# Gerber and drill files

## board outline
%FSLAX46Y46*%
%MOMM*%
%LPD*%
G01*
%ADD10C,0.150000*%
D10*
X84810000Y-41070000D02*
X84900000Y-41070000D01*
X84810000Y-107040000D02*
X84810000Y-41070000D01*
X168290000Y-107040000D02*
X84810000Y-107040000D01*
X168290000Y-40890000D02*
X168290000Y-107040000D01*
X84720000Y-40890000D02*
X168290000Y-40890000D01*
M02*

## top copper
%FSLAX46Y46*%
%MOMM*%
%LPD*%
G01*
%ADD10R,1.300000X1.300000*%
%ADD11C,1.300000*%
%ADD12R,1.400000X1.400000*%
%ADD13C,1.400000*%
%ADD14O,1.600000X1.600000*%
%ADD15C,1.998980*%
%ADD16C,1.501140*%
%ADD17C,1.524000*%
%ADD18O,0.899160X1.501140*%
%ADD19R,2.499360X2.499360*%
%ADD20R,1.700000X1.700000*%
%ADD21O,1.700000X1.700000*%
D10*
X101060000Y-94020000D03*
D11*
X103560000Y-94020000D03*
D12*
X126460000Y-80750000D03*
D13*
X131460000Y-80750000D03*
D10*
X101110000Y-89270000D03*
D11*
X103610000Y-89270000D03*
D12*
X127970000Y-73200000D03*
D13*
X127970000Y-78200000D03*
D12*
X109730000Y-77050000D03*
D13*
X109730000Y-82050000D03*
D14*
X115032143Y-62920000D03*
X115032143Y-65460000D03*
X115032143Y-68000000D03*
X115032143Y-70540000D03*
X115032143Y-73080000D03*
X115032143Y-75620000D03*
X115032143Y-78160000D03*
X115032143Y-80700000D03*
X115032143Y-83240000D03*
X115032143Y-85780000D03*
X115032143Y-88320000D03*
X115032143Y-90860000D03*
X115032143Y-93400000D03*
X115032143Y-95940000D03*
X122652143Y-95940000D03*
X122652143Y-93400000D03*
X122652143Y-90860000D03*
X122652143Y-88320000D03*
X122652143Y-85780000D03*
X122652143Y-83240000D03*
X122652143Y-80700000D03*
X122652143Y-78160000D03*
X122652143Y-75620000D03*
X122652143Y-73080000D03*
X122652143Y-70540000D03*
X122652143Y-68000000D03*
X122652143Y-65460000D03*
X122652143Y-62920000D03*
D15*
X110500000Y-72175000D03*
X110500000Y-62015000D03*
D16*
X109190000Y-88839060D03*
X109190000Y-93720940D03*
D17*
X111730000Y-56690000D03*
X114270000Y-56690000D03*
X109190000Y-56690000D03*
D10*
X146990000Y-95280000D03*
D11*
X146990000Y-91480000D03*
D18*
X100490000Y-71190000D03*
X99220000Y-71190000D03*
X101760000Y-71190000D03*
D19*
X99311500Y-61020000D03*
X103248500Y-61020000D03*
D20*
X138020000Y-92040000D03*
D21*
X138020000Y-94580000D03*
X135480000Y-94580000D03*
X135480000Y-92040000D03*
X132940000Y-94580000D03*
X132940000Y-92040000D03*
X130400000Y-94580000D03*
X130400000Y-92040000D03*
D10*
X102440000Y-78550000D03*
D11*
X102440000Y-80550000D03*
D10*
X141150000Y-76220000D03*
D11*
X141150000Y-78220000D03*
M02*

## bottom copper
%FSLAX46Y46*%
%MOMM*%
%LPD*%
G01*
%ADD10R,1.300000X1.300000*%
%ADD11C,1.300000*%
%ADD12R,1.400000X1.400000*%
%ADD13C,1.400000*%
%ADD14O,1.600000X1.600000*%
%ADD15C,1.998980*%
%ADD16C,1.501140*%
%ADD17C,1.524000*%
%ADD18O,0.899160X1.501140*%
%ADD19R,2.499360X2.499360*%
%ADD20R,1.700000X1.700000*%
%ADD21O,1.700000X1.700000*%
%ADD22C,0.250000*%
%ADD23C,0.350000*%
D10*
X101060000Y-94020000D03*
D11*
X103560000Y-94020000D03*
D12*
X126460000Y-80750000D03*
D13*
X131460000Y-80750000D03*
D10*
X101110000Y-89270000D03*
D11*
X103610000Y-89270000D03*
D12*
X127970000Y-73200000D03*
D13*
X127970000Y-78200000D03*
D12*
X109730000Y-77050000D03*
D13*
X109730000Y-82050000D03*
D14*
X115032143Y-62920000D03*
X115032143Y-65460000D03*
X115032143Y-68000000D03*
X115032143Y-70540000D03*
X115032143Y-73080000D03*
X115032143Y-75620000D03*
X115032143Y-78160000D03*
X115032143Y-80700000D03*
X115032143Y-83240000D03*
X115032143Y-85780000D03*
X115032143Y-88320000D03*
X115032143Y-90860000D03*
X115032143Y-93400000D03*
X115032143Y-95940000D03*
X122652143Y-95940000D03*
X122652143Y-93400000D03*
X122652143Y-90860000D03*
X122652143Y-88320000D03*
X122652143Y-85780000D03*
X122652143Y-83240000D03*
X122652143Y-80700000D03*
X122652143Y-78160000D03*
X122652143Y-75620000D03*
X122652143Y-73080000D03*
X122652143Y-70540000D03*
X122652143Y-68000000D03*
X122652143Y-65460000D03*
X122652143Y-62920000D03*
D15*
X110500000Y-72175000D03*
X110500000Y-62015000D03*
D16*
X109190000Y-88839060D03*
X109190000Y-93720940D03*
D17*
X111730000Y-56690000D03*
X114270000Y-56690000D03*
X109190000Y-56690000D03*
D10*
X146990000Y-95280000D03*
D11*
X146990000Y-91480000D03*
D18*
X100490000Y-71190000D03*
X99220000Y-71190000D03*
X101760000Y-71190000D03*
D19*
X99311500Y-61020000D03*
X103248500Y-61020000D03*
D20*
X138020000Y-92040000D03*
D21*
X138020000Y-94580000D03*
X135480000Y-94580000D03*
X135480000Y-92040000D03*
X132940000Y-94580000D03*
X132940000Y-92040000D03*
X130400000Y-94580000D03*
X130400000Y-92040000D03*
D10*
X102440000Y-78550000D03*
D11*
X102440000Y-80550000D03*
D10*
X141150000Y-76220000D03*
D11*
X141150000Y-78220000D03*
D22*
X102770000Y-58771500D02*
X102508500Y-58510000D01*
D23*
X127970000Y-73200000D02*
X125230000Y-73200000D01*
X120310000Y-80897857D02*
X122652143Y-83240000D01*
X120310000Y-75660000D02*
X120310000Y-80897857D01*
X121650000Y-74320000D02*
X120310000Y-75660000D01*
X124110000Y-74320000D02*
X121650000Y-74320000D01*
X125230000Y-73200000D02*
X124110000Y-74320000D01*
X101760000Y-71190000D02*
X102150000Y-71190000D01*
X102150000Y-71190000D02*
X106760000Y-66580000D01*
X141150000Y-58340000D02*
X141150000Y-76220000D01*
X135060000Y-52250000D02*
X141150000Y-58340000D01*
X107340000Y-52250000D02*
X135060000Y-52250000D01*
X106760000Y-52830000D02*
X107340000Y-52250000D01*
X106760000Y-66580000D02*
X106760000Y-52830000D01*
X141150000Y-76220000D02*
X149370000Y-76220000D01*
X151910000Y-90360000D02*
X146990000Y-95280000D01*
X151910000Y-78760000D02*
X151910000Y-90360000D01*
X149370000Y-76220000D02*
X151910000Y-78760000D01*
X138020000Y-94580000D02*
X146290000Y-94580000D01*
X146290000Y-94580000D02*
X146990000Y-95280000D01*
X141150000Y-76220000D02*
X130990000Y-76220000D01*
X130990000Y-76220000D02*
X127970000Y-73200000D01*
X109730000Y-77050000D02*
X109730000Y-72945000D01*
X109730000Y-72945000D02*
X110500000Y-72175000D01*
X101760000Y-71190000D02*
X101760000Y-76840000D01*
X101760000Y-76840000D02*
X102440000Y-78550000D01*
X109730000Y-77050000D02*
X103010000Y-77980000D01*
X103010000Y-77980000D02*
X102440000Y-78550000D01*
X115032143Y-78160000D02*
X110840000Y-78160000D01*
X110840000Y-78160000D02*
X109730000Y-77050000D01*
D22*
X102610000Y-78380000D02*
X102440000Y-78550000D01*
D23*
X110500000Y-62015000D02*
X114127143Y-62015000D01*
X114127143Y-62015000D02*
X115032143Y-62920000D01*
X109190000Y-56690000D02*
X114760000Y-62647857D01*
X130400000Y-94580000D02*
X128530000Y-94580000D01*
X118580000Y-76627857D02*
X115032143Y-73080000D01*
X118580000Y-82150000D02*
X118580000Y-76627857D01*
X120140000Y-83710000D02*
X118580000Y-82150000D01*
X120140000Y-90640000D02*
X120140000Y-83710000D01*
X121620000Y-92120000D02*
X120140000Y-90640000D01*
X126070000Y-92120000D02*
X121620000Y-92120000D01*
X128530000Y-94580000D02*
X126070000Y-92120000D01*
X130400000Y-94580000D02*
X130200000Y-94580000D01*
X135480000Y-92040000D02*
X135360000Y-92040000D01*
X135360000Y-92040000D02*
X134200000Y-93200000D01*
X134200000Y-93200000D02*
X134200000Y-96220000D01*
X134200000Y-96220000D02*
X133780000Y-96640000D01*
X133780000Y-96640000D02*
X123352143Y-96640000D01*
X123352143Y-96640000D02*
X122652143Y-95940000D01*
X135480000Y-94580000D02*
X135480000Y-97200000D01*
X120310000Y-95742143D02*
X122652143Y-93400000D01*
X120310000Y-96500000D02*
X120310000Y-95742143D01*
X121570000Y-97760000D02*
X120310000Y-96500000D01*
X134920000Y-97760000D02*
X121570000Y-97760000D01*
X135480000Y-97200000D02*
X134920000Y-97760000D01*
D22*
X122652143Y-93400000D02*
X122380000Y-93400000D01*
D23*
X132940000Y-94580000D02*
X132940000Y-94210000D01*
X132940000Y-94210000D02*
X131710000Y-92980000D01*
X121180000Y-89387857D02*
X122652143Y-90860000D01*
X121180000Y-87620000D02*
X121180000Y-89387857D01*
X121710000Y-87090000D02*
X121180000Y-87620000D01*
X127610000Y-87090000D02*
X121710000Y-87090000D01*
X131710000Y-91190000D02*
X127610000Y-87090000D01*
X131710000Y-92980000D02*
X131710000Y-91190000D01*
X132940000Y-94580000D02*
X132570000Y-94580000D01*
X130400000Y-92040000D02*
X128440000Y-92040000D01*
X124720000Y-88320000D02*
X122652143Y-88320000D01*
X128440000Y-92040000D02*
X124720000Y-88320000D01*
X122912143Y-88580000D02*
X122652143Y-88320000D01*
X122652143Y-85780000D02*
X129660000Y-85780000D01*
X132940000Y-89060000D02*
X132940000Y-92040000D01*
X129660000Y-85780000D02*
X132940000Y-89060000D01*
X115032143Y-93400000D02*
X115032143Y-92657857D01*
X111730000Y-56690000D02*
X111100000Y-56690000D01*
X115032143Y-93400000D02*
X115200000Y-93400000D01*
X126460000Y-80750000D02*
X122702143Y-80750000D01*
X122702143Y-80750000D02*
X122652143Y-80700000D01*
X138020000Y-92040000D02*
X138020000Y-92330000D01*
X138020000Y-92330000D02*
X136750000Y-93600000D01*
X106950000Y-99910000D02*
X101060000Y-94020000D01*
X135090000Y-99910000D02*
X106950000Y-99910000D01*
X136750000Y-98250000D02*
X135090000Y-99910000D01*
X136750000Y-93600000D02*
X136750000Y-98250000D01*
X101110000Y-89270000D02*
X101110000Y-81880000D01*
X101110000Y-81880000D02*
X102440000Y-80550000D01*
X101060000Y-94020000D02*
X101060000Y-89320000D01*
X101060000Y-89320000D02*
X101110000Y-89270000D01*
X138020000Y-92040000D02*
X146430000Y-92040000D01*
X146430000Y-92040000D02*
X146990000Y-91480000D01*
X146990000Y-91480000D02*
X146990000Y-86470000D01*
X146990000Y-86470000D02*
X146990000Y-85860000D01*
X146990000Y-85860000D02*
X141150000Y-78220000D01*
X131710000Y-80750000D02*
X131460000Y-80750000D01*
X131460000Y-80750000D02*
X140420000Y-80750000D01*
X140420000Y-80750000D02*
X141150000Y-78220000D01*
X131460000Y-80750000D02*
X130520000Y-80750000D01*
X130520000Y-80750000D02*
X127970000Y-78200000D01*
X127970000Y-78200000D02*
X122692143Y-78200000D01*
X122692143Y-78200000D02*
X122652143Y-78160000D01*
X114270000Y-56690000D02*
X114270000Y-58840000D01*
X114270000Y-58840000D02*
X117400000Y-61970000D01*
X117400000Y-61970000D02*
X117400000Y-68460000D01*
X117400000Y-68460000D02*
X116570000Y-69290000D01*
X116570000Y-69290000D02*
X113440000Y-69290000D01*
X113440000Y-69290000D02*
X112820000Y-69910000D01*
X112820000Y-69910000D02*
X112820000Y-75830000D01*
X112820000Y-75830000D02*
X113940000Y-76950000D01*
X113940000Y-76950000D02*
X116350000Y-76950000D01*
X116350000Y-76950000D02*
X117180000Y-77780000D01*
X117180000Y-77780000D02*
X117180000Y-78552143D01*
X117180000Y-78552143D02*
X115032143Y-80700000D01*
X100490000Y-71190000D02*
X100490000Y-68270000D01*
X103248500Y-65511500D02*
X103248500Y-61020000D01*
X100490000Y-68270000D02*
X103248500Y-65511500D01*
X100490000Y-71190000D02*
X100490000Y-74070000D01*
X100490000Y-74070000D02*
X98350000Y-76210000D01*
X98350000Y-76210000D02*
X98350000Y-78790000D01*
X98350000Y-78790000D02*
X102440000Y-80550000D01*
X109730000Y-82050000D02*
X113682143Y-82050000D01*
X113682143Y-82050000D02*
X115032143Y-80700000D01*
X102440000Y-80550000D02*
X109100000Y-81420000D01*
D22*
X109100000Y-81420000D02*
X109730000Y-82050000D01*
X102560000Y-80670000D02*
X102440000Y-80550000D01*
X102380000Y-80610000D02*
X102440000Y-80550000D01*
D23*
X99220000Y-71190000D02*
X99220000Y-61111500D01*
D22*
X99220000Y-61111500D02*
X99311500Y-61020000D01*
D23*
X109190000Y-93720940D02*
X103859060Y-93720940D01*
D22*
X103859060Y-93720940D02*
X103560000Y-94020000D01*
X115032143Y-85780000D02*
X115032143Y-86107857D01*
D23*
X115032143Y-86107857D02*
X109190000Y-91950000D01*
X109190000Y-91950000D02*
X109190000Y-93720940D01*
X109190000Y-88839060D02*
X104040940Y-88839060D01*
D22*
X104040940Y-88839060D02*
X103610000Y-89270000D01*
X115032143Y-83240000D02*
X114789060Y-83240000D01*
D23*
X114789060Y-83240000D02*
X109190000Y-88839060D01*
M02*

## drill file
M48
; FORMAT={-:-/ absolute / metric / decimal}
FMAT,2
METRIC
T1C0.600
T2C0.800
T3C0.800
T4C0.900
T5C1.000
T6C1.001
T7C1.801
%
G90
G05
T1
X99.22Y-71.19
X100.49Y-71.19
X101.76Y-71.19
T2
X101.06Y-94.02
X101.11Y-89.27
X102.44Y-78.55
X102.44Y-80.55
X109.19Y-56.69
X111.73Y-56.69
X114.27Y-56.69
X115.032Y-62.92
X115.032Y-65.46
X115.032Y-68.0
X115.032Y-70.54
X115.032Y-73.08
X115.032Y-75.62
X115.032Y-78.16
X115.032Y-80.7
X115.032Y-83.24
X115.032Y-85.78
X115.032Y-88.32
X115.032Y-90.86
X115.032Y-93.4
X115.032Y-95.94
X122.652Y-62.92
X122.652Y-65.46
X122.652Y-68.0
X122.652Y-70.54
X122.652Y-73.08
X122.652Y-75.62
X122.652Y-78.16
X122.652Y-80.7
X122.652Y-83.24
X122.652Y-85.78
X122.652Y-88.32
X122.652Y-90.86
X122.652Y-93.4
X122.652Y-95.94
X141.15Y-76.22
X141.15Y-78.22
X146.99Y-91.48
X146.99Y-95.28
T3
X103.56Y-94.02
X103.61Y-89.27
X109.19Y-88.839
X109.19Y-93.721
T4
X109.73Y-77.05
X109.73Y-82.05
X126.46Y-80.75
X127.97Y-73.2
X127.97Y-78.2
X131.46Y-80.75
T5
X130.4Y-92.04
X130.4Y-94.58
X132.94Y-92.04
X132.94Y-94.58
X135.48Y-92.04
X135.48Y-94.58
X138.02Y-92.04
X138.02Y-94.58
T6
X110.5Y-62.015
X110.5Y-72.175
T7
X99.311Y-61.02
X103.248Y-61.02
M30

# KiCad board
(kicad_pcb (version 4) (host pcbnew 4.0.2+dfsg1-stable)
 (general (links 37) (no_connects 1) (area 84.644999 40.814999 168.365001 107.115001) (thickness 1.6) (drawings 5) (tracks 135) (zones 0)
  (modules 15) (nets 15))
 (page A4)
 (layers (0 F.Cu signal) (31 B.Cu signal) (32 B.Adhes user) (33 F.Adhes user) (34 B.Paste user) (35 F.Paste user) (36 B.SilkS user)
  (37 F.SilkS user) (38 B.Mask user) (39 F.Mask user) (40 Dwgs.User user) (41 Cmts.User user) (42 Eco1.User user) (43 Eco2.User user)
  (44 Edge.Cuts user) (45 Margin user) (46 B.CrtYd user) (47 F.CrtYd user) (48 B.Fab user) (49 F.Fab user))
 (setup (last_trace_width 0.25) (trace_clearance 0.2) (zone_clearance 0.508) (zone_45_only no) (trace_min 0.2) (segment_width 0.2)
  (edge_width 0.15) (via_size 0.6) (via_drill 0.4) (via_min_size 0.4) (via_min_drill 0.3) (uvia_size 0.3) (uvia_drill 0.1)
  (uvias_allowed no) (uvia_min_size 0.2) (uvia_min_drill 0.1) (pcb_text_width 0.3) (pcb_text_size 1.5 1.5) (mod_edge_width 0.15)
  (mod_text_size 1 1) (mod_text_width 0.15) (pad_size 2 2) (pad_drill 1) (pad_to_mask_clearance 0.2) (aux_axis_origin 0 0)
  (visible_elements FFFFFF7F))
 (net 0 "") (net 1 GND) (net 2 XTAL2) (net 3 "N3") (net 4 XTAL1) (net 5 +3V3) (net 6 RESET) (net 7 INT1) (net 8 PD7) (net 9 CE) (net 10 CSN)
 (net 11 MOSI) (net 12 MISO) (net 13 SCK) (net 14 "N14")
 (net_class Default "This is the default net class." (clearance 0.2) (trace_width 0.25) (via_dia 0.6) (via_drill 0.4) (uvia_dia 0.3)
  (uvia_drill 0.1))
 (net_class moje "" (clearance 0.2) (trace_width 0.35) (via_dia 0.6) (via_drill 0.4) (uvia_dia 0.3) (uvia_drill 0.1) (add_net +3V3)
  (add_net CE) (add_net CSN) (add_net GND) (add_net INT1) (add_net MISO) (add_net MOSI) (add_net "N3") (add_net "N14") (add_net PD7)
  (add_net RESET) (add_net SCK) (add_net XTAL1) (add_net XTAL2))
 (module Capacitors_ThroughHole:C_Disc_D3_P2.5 (layer F.Cu) (at 101.06 94.02)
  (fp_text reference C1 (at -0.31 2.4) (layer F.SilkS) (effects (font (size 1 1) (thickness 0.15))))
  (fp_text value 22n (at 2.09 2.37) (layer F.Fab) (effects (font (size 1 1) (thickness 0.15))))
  (pad 1 thru_hole rect (at 0 0) (size 1.3 1.3) (drill 0.8) (layers *.Cu *.Mask F.SilkS) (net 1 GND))
  (pad 2 thru_hole circle (at 2.5 0) (size 1.3 1.3) (drill 0.8001) (layers *.Cu *.Mask F.SilkS) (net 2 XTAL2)))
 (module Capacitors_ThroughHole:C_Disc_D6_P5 (layer F.Cu) (at 126.46 80.75)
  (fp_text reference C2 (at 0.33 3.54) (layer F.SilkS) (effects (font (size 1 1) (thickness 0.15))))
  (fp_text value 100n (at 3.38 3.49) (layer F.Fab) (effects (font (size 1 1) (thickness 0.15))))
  (pad 1 thru_hole rect (at 0 0) (size 1.4 1.4) (drill 0.9) (layers *.Cu *.Mask F.SilkS) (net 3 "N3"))
  (pad 2 thru_hole circle (at 5 0) (size 1.4 1.4) (drill 0.9) (layers *.Cu *.Mask F.SilkS) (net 1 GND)))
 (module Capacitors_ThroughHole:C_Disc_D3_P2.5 (layer F.Cu) (at 101.11 89.27)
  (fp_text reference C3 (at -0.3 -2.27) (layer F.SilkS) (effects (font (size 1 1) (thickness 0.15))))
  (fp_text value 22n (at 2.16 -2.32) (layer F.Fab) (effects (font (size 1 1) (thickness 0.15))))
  (pad 1 thru_hole rect (at 0 0) (size 1.3 1.3) (drill 0.8) (layers *.Cu *.Mask F.SilkS) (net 1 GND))
  (pad 2 thru_hole circle (at 2.5 0) (size 1.3 1.3) (drill 0.8001) (layers *.Cu *.Mask F.SilkS) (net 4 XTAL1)))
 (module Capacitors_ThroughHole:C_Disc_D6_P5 (layer F.Cu) (at 127.97 73.2 270)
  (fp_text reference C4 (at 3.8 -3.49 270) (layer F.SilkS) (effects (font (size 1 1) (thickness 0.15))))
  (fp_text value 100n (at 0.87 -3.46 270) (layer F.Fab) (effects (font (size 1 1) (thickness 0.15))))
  (pad 1 thru_hole rect (at 0 0 270) (size 1.4 1.4) (drill 0.9) (layers *.Cu *.Mask F.SilkS) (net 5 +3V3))
  (pad 2 thru_hole circle (at 5 0 270) (size 1.4 1.4) (drill 0.9) (layers *.Cu *.Mask F.SilkS) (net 1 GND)))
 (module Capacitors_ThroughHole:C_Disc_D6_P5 (layer F.Cu) (at 109.73 77.05 270)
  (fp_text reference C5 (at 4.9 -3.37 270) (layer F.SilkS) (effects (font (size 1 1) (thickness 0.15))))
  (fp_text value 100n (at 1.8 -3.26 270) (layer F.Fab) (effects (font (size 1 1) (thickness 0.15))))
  (pad 1 thru_hole rect (at 0 0 270) (size 1.4 1.4) (drill 0.9) (layers *.Cu *.Mask F.SilkS) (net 5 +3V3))
  (pad 2 thru_hole circle (at 5 0 270) (size 1.4 1.4) (drill 0.9) (layers *.Cu *.Mask F.SilkS) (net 1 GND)))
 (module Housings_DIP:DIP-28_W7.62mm (layer F.Cu) (at 115.032143 62.92)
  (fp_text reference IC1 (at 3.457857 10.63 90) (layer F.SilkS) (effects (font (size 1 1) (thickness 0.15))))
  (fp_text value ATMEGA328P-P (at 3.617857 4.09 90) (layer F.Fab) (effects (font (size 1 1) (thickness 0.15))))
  (pad 1 thru_hole oval (at 0 0) (size 1.6 1.6) (drill 0.8) (layers *.Cu *.Mask F.SilkS) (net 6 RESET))
  (pad 2 thru_hole oval (at 0 2.54) (size 1.6 1.6) (drill 0.8) (layers *.Cu *.Mask F.SilkS))
  (pad 3 thru_hole oval (at 0 5.08) (size 1.6 1.6) (drill 0.8) (layers *.Cu *.Mask F.SilkS))
  (pad 4 thru_hole oval (at 0 7.62) (size 1.6 1.6) (drill 0.8) (layers *.Cu *.Mask F.SilkS))
  (pad 5 thru_hole oval (at 0 10.16) (size 1.6 1.6) (drill 0.8) (layers *.Cu *.Mask F.SilkS) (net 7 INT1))
  (pad 6 thru_hole oval (at 0 12.7) (size 1.6 1.6) (drill 0.8) (layers *.Cu *.Mask F.SilkS))
  (pad 7 thru_hole oval (at 0 15.24) (size 1.6 1.6) (drill 0.8) (layers *.Cu *.Mask F.SilkS) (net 5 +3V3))
  (pad 8 thru_hole oval (at 0 17.78) (size 1.6 1.6) (drill 0.8) (layers *.Cu *.Mask F.SilkS) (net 1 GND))
  (pad 9 thru_hole oval (at 0 20.32) (size 1.6 1.6) (drill 0.8) (layers *.Cu *.Mask F.SilkS) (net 4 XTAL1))
  (pad 10 thru_hole oval (at 0 22.86) (size 1.6 1.6) (drill 0.8) (layers *.Cu *.Mask F.SilkS) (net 2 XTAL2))
  (pad 11 thru_hole oval (at 0 25.4) (size 1.6 1.6) (drill 0.8) (layers *.Cu *.Mask F.SilkS))
  (pad 12 thru_hole oval (at 0 27.94) (size 1.6 1.6) (drill 0.8) (layers *.Cu *.Mask F.SilkS))
  (pad 13 thru_hole oval (at 0 30.48) (size 1.6 1.6) (drill 0.8) (layers *.Cu *.Mask F.SilkS) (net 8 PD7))
  (pad 14 thru_hole oval (at 0 33.02) (size 1.6 1.6) (drill 0.8) (layers *.Cu *.Mask F.SilkS))
  (pad 15 thru_hole oval (at 7.62 33.02) (size 1.6 1.6) (drill 0.8) (layers *.Cu *.Mask F.SilkS) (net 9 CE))
  (pad 16 thru_hole oval (at 7.62 30.48) (size 1.6 1.6) (drill 0.8) (layers *.Cu *.Mask F.SilkS) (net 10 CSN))
  (pad 17 thru_hole oval (at 7.62 27.94) (size 1.6 1.6) (drill 0.8) (layers *.Cu *.Mask F.SilkS) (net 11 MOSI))
  (pad 18 thru_hole oval (at 7.62 25.4) (size 1.6 1.6) (drill 0.8) (layers *.Cu *.Mask F.SilkS) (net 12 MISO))
  (pad 19 thru_hole oval (at 7.62 22.86) (size 1.6 1.6) (drill 0.8) (layers *.Cu *.Mask F.SilkS) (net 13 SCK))
  (pad 20 thru_hole oval (at 7.62 20.32) (size 1.6 1.6) (drill 0.8) (layers *.Cu *.Mask F.SilkS) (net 5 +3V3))
  (pad 21 thru_hole oval (at 7.62 17.78) (size 1.6 1.6) (drill 0.8) (layers *.Cu *.Mask F.SilkS) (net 3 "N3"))
  (pad 22 thru_hole oval (at 7.62 15.24) (size 1.6 1.6) (drill 0.8) (layers *.Cu *.Mask F.SilkS) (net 1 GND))
  (pad 23 thru_hole oval (at 7.62 12.7) (size 1.6 1.6) (drill 0.8) (layers *.Cu *.Mask F.SilkS))
  (pad 24 thru_hole oval (at 7.62 10.16) (size 1.6 1.6) (drill 0.8) (layers *.Cu *.Mask F.SilkS))
  (pad 25 thru_hole oval (at 7.62 7.62) (size 1.6 1.6) (drill 0.8) (layers *.Cu *.Mask F.SilkS))
  (pad 26 thru_hole oval (at 7.62 5.08) (size 1.6 1.6) (drill 0.8) (layers *.Cu *.Mask F.SilkS))
  (pad 27 thru_hole oval (at 7.62 2.54) (size 1.6 1.6) (drill 0.8) (layers *.Cu *.Mask F.SilkS))
  (pad 28 thru_hole oval (at 7.62 0) (size 1.6 1.6) (drill 0.8) (layers *.Cu *.Mask F.SilkS)))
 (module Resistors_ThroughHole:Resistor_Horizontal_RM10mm (layer F.Cu) (at 110.5 72.175 90)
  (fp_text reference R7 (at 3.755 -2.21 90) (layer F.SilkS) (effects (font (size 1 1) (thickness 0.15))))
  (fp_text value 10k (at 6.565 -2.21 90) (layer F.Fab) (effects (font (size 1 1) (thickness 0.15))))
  (pad 1 thru_hole circle (at 0 0 90) (size 1.99898 1.99898) (drill 1.00076) (layers *.Cu *.SilkS *.Mask) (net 5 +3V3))
  (pad 2 thru_hole circle (at 10.16 0 90) (size 1.99898 1.99898) (drill 1.00076) (layers *.Cu *.SilkS *.Mask) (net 6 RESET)))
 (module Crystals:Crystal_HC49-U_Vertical (layer F.Cu) (at 109.19 91.28 270)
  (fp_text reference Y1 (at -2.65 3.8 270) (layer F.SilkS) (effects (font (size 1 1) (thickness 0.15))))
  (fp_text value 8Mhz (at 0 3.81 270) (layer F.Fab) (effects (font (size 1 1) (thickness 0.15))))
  (pad 1 thru_hole circle (at -2.44094 0 270) (size 1.50114 1.50114) (drill 0.8001) (layers *.Cu *.Mask F.SilkS) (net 4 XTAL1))
  (pad 2 thru_hole circle (at 2.44094 0 270) (size 1.50114 1.50114) (drill 0.8001) (layers *.Cu *.Mask F.SilkS) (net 2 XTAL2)))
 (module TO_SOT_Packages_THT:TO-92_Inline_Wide (layer F.Cu) (at 109.19 56.69)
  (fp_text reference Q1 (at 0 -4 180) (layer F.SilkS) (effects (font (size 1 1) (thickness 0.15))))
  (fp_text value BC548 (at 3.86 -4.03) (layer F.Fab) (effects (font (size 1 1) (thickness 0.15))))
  (pad 2 thru_hole circle (at 2.54 0 90) (size 1.524 1.524) (drill 0.8) (layers *.Cu *.Mask F.SilkS) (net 8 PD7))
  (pad 3 thru_hole circle (at 5.08 0 90) (size 1.524 1.524) (drill 0.8) (layers *.Cu *.Mask F.SilkS) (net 1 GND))
  (pad 1 thru_hole circle (at 0 0 90) (size 1.524 1.524) (drill 0.8) (layers *.Cu *.Mask F.SilkS) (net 6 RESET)))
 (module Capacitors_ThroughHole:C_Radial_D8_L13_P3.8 (layer F.Cu) (at 146.99 95.28 90)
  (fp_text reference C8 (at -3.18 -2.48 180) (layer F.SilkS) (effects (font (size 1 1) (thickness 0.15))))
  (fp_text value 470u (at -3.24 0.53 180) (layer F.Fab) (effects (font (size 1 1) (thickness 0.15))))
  (pad 1 thru_hole rect (at 0 0 90) (size 1.3 1.3) (drill 0.8) (layers *.Cu *.Mask F.SilkS) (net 5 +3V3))
  (pad 2 thru_hole circle (at 3.8 0 90) (size 1.3 1.3) (drill 0.8) (layers *.Cu *.Mask F.SilkS) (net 1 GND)))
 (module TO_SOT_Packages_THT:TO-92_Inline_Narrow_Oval (layer F.Cu) (at 101.76 71.19 180)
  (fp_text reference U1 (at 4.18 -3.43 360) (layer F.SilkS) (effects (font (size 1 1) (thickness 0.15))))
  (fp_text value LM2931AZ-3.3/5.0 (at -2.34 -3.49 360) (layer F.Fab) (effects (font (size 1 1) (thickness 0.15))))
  (pad 2 thru_hole oval (at 1.27 0) (size 0.89916 1.50114) (drill 0.6) (layers *.Cu *.Mask F.SilkS) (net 1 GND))
  (pad 3 thru_hole oval (at 2.54 0) (size 0.89916 1.50114) (drill 0.6) (layers *.Cu *.Mask F.SilkS) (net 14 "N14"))
  (pad 1 thru_hole oval (at 0 0) (size 0.89916 1.50114) (drill 0.6) (layers *.Cu *.Mask F.SilkS) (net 5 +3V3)))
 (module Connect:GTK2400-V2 (layer F.Cu) (at 101.28 61.02 180)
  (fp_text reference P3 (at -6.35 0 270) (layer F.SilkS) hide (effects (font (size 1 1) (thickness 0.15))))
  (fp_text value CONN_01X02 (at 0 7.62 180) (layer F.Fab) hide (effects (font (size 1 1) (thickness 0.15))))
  (pad 2 thru_hole rect (at 1.9685 0 180) (size 2.49936 2.49936) (drill 1.80086) (layers *.Cu *.Mask F.SilkS) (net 14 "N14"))
  (pad 1 thru_hole rect (at -1.9685 0 180) (size 2.49936 2.49936) (drill 1.80086) (layers *.Cu *.Mask F.SilkS) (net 1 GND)))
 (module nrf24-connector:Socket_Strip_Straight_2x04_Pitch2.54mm (layer F.Cu) (at 138.02 94.58 270)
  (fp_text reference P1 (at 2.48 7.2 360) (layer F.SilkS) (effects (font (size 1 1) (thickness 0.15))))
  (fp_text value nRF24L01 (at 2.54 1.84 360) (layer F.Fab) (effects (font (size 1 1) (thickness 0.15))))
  (pad 1 thru_hole rect (at -2.54 0 270) (size 1.7 1.7) (drill 1) (layers *.Cu *.Mask) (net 1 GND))
  (pad 2 thru_hole oval (at 0 0 270) (size 1.7 1.7) (drill 1) (layers *.Cu *.Mask) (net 5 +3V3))
  (pad 4 thru_hole oval (at 0 2.54 270) (size 1.7 1.7) (drill 1) (layers *.Cu *.Mask) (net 10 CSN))
  (pad 3 thru_hole oval (at -2.54 2.54 270) (size 1.7 1.7) (drill 1) (layers *.Cu *.Mask) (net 9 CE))
  (pad 6 thru_hole oval (at 0 5.08 270) (size 1.7 1.7) (drill 1) (layers *.Cu *.Mask) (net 11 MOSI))
  (pad 5 thru_hole oval (at -2.54 5.08 270) (size 1.7 1.7) (drill 1) (layers *.Cu *.Mask) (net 13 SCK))
  (pad 8 thru_hole oval (at 0 7.62 270) (size 1.7 1.7) (drill 1) (layers *.Cu *.Mask) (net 7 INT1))
  (pad 7 thru_hole oval (at -2.54 7.62 270) (size 1.7 1.7) (drill 1) (layers *.Cu *.Mask) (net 12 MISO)))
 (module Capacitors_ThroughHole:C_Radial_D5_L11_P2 (layer F.Cu) (at 102.44 78.55 270)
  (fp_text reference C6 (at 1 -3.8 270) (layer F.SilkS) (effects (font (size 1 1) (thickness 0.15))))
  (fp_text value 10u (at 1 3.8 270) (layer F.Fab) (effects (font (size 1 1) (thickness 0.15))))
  (pad 1 thru_hole rect (at 0 0 270) (size 1.3 1.3) (drill 0.8) (layers *.Cu *.Mask F.SilkS) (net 5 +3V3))
  (pad 2 thru_hole circle (at 2 0 270) (size 1.3 1.3) (drill 0.8) (layers *.Cu *.Mask F.SilkS) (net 1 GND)))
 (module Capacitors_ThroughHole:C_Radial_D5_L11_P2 (layer F.Cu) (at 141.15 76.22 270)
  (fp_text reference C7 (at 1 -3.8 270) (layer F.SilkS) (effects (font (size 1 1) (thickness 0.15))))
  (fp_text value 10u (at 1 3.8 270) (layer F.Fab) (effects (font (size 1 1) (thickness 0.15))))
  (pad 1 thru_hole rect (at 0 0 270) (size 1.3 1.3) (drill 0.8) (layers *.Cu *.Mask F.SilkS) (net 5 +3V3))
  (pad 2 thru_hole circle (at 2 0 270) (size 1.3 1.3) (drill 0.8) (layers *.Cu *.Mask F.SilkS) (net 1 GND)))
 (gr_line (start 84.81 41.07) (end 84.9 41.07) (angle 90) (layer Edge.Cuts) (width 0.15))
 (gr_line (start 84.81 107.04) (end 84.81 41.07) (angle 90) (layer Edge.Cuts) (width 0.15))
 (gr_line (start 168.29 107.04) (end 84.81 107.04) (angle 90) (layer Edge.Cuts) (width 0.15))
 (gr_line (start 168.29 40.89) (end 168.29 107.04) (angle 90) (layer Edge.Cuts) (width 0.15))
 (gr_line (start 84.72 40.89) (end 168.29 40.89) (angle 90) (layer Edge.Cuts) (width 0.15))
 (segment (start 102.77 58.7715) (end 102.5085 58.51) (width 0.25) (layer B.Cu) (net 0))
 (segment (start 127.97 73.2) (end 125.23 73.2) (width 0.35) (layer B.Cu) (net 5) (status 400000))
 (segment (start 120.31 80.897857) (end 122.652143 83.24) (width 0.35) (layer B.Cu) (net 5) (status 800000))
 (segment (start 120.31 75.66) (end 120.31 80.897857) (width 0.35) (layer B.Cu) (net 5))
 (segment (start 121.65 74.32) (end 120.31 75.66) (width 0.35) (layer B.Cu) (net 5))
 (segment (start 124.11 74.32) (end 121.65 74.32) (width 0.35) (layer B.Cu) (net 5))
 (segment (start 125.23 73.2) (end 124.11 74.32) (width 0.35) (layer B.Cu) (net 5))
 (segment (start 101.76 71.19) (end 102.15 71.19) (width 0.35) (layer B.Cu) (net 5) (status C00000))
 (segment (start 102.15 71.19) (end 106.76 66.58) (width 0.35) (layer B.Cu) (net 5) (status 400000))
 (segment (start 141.15 58.34) (end 141.15 76.22) (width 0.35) (layer B.Cu) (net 5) (status 800000))
 (segment (start 135.06 52.25) (end 141.15 58.34) (width 0.35) (layer B.Cu) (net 5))
 (segment (start 107.34 52.25) (end 135.06 52.25) (width 0.35) (layer B.Cu) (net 5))
 (segment (start 106.76 52.83) (end 107.34 52.25) (width 0.35) (layer B.Cu) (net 5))
 (segment (start 106.76 66.58) (end 106.76 52.83) (width 0.35) (layer B.Cu) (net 5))
 (segment (start 141.15 76.22) (end 149.37 76.22) (width 0.35) (layer B.Cu) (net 5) (status 400000))
 (segment (start 151.91 90.36) (end 146.99 95.28) (width 0.35) (layer B.Cu) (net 5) (status 800000))
 (segment (start 151.91 78.76) (end 151.91 90.36) (width 0.35) (layer B.Cu) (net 5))
 (segment (start 149.37 76.22) (end 151.91 78.76) (width 0.35) (layer B.Cu) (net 5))
 (segment (start 138.02 94.58) (end 146.29 94.58) (width 0.35) (layer B.Cu) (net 5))
 (segment (start 146.29 94.58) (end 146.99 95.28) (width 0.35) (layer B.Cu) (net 5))
 (segment (start 141.15 76.22) (end 130.99 76.22) (width 0.35) (layer B.Cu) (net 5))
 (segment (start 130.99 76.22) (end 127.97 73.2) (width 0.35) (layer B.Cu) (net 5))
 (segment (start 109.73 77.05) (end 109.73 72.945) (width 0.35) (layer B.Cu) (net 5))
 (segment (start 109.73 72.945) (end 110.5 72.175) (width 0.35) (layer B.Cu) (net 5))
 (segment (start 101.76 71.19) (end 101.76 76.84) (width 0.35) (layer B.Cu) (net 5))
 (segment (start 101.76 76.84) (end 102.44 78.55) (width 0.35) (layer B.Cu) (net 5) (status 20))
 (segment (start 109.73 77.05) (end 103.01 77.98) (width 0.35) (layer B.Cu) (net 5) (status 20))
 (segment (start 103.01 77.98) (end 102.44 78.55) (width 0.35) (layer B.Cu) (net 5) (status 30))
 (segment (start 115.032143 78.16) (end 110.84 78.16) (width 0.35) (layer B.Cu) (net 5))
 (segment (start 110.84 78.16) (end 109.73 77.05) (width 0.35) (layer B.Cu) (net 5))
 (segment (start 102.61 78.38) (end 102.44 78.55) (width 0.25) (layer B.Cu) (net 5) (status 30))
 (segment (start 110.5 62.015) (end 114.127143 62.015) (width 0.35) (layer B.Cu) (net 6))
 (segment (start 114.127143 62.015) (end 115.032143 62.92) (width 0.35) (layer B.Cu) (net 6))
 (segment (start 109.19 56.69) (end 114.76 62.647857) (width 0.35) (layer B.Cu) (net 6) (status 10))
 (segment (start 130.4 94.58) (end 128.53 94.58) (width 0.35) (layer B.Cu) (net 7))
 (segment (start 118.58 76.627857) (end 115.032143 73.08) (width 0.35) (layer B.Cu) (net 7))
 (segment (start 118.58 82.15) (end 118.58 76.627857) (width 0.35) (layer B.Cu) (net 7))
 (segment (start 120.14 83.71) (end 118.58 82.15) (width 0.35) (layer B.Cu) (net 7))
 (segment (start 120.14 90.64) (end 120.14 83.71) (width 0.35) (layer B.Cu) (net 7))
 (segment (start 121.62 92.12) (end 120.14 90.64) (width 0.35) (layer B.Cu) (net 7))
 (segment (start 126.07 92.12) (end 121.62 92.12) (width 0.35) (layer B.Cu) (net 7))
 (segment (start 128.53 94.58) (end 126.07 92.12) (width 0.35) (layer B.Cu) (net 7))
 (segment (start 130.4 94.58) (end 130.2 94.58) (width 0.35) (layer B.Cu) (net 7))
 (segment (start 135.48 92.04) (end 135.36 92.04) (width 0.35) (layer B.Cu) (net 9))
 (segment (start 135.36 92.04) (end 134.2 93.2) (width 0.35) (layer B.Cu) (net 9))
 (segment (start 134.2 93.2) (end 134.2 96.22) (width 0.35) (layer B.Cu) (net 9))
 (segment (start 134.2 96.22) (end 133.78 96.64) (width 0.35) (layer B.Cu) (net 9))
 (segment (start 133.78 96.64) (end 123.352143 96.64) (width 0.35) (layer B.Cu) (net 9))
 (segment (start 123.352143 96.64) (end 122.652143 95.94) (width 0.35) (layer B.Cu) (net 9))
 (segment (start 135.48 94.58) (end 135.48 97.2) (width 0.35) (layer B.Cu) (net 10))
 (segment (start 120.31 95.742143) (end 122.652143 93.4) (width 0.35) (layer B.Cu) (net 10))
 (segment (start 120.31 96.5) (end 120.31 95.742143) (width 0.35) (layer B.Cu) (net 10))
 (segment (start 121.57 97.76) (end 120.31 96.5) (width 0.35) (layer B.Cu) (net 10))
 (segment (start 134.92 97.76) (end 121.57 97.76) (width 0.35) (layer B.Cu) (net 10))
 (segment (start 135.48 97.2) (end 134.92 97.76) (width 0.35) (layer B.Cu) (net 10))
 (segment (start 122.652143 93.4) (end 122.38 93.4) (width 0.25) (layer B.Cu) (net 10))
 (segment (start 132.94 94.58) (end 132.94 94.21) (width 0.35) (layer B.Cu) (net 11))
 (segment (start 132.94 94.21) (end 131.71 92.98) (width 0.35) (layer B.Cu) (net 11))
 (segment (start 121.18 89.387857) (end 122.652143 90.86) (width 0.35) (layer B.Cu) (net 11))
 (segment (start 121.18 87.62) (end 121.18 89.387857) (width 0.35) (layer B.Cu) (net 11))
 (segment (start 121.71 87.09) (end 121.18 87.62) (width 0.35) (layer B.Cu) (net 11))
 (segment (start 127.61 87.09) (end 121.71 87.09) (width 0.35) (layer B.Cu) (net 11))
 (segment (start 131.71 91.19) (end 127.61 87.09) (width 0.35) (layer B.Cu) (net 11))
 (segment (start 131.71 92.98) (end 131.71 91.19) (width 0.35) (layer B.Cu) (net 11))
 (segment (start 132.94 94.58) (end 132.57 94.58) (width 0.35) (layer B.Cu) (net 11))
 (segment (start 130.4 92.04) (end 128.44 92.04) (width 0.35) (layer B.Cu) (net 12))
 (segment (start 124.72 88.32) (end 122.652143 88.32) (width 0.35) (layer B.Cu) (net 12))
 (segment (start 128.44 92.04) (end 124.72 88.32) (width 0.35) (layer B.Cu) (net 12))
 (segment (start 122.912143 88.58) (end 122.652143 88.32) (width 0.35) (layer B.Cu) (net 12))
 (segment (start 122.652143 85.78) (end 129.66 85.78) (width 0.35) (layer B.Cu) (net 13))
 (segment (start 132.94 89.06) (end 132.94 92.04) (width 0.35) (layer B.Cu) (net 13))
 (segment (start 129.66 85.78) (end 132.94 89.06) (width 0.35) (layer B.Cu) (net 13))
 (segment (start 115.032143 93.4) (end 115.032143 92.657857) (width 0.35) (layer B.Cu) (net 8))
 (segment (start 111.73 56.69) (end 111.1 56.69) (width 0.35) (layer B.Cu) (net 8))
 (segment (start 115.032143 93.4) (end 115.2 93.4) (width 0.35) (layer B.Cu) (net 8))
 (segment (start 126.46 80.75) (end 122.702143 80.75) (width 0.35) (layer B.Cu) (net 3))
 (segment (start 122.702143 80.75) (end 122.652143 80.7) (width 0.35) (layer B.Cu) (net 3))
 (segment (start 138.02 92.04) (end 138.02 92.33) (width 0.35) (layer B.Cu) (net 1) (status C00000))
 (segment (start 138.02 92.33) (end 136.75 93.6) (width 0.35) (layer B.Cu) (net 1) (status 400000))
 (segment (start 106.95 99.91) (end 101.06 94.02) (width 0.35) (layer B.Cu) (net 1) (status 800000))
 (segment (start 135.09 99.91) (end 106.95 99.91) (width 0.35) (layer B.Cu) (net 1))
 (segment (start 136.75 98.25) (end 135.09 99.91) (width 0.35) (layer B.Cu) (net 1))
 (segment (start 136.75 93.6) (end 136.75 98.25) (width 0.35) (layer B.Cu) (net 1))
 (segment (start 101.11 89.27) (end 101.11 81.88) (width 0.35) (layer B.Cu) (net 1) (status 400000))
 (segment (start 101.11 81.88) (end 102.44 80.55) (width 0.35) (layer B.Cu) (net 1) (status 800000))
 (segment (start 101.06 94.02) (end 101.06 89.32) (width 0.35) (layer B.Cu) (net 1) (status C00000))
 (segment (start 101.06 89.32) (end 101.11 89.27) (width 0.35) (layer B.Cu) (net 1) (status C00000))
 (segment (start 138.02 92.04) (end 146.43 92.04) (width 0.35) (layer B.Cu) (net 1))
 (segment (start 146.43 92.04) (end 146.99 91.48) (width 0.35) (layer B.Cu) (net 1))
 (segment (start 146.99 91.48) (end 146.99 86.47) (width 0.35) (layer B.Cu) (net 1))
 (segment (start 146.99 86.47) (end 146.99 85.86) (width 0.35) (layer B.Cu) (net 1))
 (segment (start 146.99 85.86) (end 141.15 78.22) (width 0.35) (layer B.Cu) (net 1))
 (segment (start 131.71 80.75) (end 131.46 80.75) (width 0.35) (layer B.Cu) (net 1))
 (segment (start 131.46 80.75) (end 140.42 80.75) (width 0.35) (layer B.Cu) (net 1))
 (segment (start 140.42 80.75) (end 141.15 78.22) (width 0.35) (layer B.Cu) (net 1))
 (segment (start 131.46 80.75) (end 130.52 80.75) (width 0.35) (layer B.Cu) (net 1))
 (segment (start 130.52 80.75) (end 127.97 78.2) (width 0.35) (layer B.Cu) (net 1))
 (segment (start 127.97 78.2) (end 122.692143 78.2) (width 0.35) (layer B.Cu) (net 1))
 (segment (start 122.692143 78.2) (end 122.652143 78.16) (width 0.35) (layer B.Cu) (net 1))
 (segment (start 114.27 56.69) (end 114.27 58.84) (width 0.35) (layer B.Cu) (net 1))
 (segment (start 114.27 58.84) (end 117.4 61.97) (width 0.35) (layer B.Cu) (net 1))
 (segment (start 117.4 61.97) (end 117.4 68.46) (width 0.35) (layer B.Cu) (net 1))
 (segment (start 117.4 68.46) (end 116.57 69.29) (width 0.35) (layer B.Cu) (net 1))
 (segment (start 116.57 69.29) (end 113.44 69.29) (width 0.35) (layer B.Cu) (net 1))
 (segment (start 113.44 69.29) (end 112.82 69.91) (width 0.35) (layer B.Cu) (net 1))
 (segment (start 112.82 69.91) (end 112.82 75.83) (width 0.35) (layer B.Cu) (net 1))
 (segment (start 112.82 75.83) (end 113.94 76.95) (width 0.35) (layer B.Cu) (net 1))
 (segment (start 113.94 76.95) (end 116.35 76.95) (width 0.35) (layer B.Cu) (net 1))
 (segment (start 116.35 76.95) (end 117.18 77.78) (width 0.35) (layer B.Cu) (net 1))
 (segment (start 117.18 77.78) (end 117.18 78.552143) (width 0.35) (layer B.Cu) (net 1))
 (segment (start 117.18 78.552143) (end 115.032143 80.7) (width 0.35) (layer B.Cu) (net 1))
 (segment (start 100.49 71.19) (end 100.49 68.27) (width 0.35) (layer B.Cu) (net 1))
 (segment (start 103.2485 65.5115) (end 103.2485 61.02) (width 0.35) (layer B.Cu) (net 1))
 (segment (start 100.49 68.27) (end 103.2485 65.5115) (width 0.35) (layer B.Cu) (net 1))
 (segment (start 100.49 71.19) (end 100.49 74.07) (width 0.35) (layer B.Cu) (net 1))
 (segment (start 100.49 74.07) (end 98.35 76.21) (width 0.35) (layer B.Cu) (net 1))
 (segment (start 98.35 76.21) (end 98.35 78.79) (width 0.35) (layer B.Cu) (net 1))
 (segment (start 98.35 78.79) (end 102.44 80.55) (width 0.35) (layer B.Cu) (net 1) (status 20))
 (segment (start 109.73 82.05) (end 113.682143 82.05) (width 0.35) (layer B.Cu) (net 1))
 (segment (start 113.682143 82.05) (end 115.032143 80.7) (width 0.35) (layer B.Cu) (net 1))
 (segment (start 102.44 80.55) (end 109.1 81.42) (width 0.35) (layer B.Cu) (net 1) (status 10))
 (segment (start 109.1 81.42) (end 109.73 82.05) (width 0.25) (layer B.Cu) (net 1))
 (segment (start 102.56 80.67) (end 102.44 80.55) (width 0.25) (layer B.Cu) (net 1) (status 30))
 (segment (start 102.38 80.61) (end 102.44 80.55) (width 0.25) (layer B.Cu) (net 1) (status 30))
 (segment (start 99.22 71.19) (end 99.22 61.1115) (width 0.35) (layer B.Cu) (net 14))
 (segment (start 99.22 61.1115) (end 99.3115 61.02) (width 0.25) (layer B.Cu) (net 14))
 (segment (start 109.19 93.72094) (end 103.85906 93.72094) (width 0.35) (layer B.Cu) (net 2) (status C00000))
 (segment (start 103.85906 93.72094) (end 103.56 94.02) (width 0.25) (layer B.Cu) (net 2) (status C00000))
 (segment (start 115.032143 85.78) (end 115.032143 86.107857) (width 0.25) (layer B.Cu) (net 2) (status C00000))
 (segment (start 115.032143 86.107857) (end 109.19 91.95) (width 0.35) (layer B.Cu) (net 2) (status 400000))
 (segment (start 109.19 91.95) (end 109.19 93.72094) (width 0.35) (layer B.Cu) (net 2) (status 800000))
 (segment (start 109.19 88.83906) (end 104.04094 88.83906) (width 0.35) (layer B.Cu) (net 4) (status C00000))
 (segment (start 104.04094 88.83906) (end 103.61 89.27) (width 0.25) (layer B.Cu) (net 4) (status C00000))
 (segment (start 115.032143 83.24) (end 114.78906 83.24) (width 0.25) (layer B.Cu) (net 4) (status C00000))
 (segment (start 114.78906 83.24) (end 109.19 88.83906) (width 0.35) (layer B.Cu) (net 4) (status C00000)))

